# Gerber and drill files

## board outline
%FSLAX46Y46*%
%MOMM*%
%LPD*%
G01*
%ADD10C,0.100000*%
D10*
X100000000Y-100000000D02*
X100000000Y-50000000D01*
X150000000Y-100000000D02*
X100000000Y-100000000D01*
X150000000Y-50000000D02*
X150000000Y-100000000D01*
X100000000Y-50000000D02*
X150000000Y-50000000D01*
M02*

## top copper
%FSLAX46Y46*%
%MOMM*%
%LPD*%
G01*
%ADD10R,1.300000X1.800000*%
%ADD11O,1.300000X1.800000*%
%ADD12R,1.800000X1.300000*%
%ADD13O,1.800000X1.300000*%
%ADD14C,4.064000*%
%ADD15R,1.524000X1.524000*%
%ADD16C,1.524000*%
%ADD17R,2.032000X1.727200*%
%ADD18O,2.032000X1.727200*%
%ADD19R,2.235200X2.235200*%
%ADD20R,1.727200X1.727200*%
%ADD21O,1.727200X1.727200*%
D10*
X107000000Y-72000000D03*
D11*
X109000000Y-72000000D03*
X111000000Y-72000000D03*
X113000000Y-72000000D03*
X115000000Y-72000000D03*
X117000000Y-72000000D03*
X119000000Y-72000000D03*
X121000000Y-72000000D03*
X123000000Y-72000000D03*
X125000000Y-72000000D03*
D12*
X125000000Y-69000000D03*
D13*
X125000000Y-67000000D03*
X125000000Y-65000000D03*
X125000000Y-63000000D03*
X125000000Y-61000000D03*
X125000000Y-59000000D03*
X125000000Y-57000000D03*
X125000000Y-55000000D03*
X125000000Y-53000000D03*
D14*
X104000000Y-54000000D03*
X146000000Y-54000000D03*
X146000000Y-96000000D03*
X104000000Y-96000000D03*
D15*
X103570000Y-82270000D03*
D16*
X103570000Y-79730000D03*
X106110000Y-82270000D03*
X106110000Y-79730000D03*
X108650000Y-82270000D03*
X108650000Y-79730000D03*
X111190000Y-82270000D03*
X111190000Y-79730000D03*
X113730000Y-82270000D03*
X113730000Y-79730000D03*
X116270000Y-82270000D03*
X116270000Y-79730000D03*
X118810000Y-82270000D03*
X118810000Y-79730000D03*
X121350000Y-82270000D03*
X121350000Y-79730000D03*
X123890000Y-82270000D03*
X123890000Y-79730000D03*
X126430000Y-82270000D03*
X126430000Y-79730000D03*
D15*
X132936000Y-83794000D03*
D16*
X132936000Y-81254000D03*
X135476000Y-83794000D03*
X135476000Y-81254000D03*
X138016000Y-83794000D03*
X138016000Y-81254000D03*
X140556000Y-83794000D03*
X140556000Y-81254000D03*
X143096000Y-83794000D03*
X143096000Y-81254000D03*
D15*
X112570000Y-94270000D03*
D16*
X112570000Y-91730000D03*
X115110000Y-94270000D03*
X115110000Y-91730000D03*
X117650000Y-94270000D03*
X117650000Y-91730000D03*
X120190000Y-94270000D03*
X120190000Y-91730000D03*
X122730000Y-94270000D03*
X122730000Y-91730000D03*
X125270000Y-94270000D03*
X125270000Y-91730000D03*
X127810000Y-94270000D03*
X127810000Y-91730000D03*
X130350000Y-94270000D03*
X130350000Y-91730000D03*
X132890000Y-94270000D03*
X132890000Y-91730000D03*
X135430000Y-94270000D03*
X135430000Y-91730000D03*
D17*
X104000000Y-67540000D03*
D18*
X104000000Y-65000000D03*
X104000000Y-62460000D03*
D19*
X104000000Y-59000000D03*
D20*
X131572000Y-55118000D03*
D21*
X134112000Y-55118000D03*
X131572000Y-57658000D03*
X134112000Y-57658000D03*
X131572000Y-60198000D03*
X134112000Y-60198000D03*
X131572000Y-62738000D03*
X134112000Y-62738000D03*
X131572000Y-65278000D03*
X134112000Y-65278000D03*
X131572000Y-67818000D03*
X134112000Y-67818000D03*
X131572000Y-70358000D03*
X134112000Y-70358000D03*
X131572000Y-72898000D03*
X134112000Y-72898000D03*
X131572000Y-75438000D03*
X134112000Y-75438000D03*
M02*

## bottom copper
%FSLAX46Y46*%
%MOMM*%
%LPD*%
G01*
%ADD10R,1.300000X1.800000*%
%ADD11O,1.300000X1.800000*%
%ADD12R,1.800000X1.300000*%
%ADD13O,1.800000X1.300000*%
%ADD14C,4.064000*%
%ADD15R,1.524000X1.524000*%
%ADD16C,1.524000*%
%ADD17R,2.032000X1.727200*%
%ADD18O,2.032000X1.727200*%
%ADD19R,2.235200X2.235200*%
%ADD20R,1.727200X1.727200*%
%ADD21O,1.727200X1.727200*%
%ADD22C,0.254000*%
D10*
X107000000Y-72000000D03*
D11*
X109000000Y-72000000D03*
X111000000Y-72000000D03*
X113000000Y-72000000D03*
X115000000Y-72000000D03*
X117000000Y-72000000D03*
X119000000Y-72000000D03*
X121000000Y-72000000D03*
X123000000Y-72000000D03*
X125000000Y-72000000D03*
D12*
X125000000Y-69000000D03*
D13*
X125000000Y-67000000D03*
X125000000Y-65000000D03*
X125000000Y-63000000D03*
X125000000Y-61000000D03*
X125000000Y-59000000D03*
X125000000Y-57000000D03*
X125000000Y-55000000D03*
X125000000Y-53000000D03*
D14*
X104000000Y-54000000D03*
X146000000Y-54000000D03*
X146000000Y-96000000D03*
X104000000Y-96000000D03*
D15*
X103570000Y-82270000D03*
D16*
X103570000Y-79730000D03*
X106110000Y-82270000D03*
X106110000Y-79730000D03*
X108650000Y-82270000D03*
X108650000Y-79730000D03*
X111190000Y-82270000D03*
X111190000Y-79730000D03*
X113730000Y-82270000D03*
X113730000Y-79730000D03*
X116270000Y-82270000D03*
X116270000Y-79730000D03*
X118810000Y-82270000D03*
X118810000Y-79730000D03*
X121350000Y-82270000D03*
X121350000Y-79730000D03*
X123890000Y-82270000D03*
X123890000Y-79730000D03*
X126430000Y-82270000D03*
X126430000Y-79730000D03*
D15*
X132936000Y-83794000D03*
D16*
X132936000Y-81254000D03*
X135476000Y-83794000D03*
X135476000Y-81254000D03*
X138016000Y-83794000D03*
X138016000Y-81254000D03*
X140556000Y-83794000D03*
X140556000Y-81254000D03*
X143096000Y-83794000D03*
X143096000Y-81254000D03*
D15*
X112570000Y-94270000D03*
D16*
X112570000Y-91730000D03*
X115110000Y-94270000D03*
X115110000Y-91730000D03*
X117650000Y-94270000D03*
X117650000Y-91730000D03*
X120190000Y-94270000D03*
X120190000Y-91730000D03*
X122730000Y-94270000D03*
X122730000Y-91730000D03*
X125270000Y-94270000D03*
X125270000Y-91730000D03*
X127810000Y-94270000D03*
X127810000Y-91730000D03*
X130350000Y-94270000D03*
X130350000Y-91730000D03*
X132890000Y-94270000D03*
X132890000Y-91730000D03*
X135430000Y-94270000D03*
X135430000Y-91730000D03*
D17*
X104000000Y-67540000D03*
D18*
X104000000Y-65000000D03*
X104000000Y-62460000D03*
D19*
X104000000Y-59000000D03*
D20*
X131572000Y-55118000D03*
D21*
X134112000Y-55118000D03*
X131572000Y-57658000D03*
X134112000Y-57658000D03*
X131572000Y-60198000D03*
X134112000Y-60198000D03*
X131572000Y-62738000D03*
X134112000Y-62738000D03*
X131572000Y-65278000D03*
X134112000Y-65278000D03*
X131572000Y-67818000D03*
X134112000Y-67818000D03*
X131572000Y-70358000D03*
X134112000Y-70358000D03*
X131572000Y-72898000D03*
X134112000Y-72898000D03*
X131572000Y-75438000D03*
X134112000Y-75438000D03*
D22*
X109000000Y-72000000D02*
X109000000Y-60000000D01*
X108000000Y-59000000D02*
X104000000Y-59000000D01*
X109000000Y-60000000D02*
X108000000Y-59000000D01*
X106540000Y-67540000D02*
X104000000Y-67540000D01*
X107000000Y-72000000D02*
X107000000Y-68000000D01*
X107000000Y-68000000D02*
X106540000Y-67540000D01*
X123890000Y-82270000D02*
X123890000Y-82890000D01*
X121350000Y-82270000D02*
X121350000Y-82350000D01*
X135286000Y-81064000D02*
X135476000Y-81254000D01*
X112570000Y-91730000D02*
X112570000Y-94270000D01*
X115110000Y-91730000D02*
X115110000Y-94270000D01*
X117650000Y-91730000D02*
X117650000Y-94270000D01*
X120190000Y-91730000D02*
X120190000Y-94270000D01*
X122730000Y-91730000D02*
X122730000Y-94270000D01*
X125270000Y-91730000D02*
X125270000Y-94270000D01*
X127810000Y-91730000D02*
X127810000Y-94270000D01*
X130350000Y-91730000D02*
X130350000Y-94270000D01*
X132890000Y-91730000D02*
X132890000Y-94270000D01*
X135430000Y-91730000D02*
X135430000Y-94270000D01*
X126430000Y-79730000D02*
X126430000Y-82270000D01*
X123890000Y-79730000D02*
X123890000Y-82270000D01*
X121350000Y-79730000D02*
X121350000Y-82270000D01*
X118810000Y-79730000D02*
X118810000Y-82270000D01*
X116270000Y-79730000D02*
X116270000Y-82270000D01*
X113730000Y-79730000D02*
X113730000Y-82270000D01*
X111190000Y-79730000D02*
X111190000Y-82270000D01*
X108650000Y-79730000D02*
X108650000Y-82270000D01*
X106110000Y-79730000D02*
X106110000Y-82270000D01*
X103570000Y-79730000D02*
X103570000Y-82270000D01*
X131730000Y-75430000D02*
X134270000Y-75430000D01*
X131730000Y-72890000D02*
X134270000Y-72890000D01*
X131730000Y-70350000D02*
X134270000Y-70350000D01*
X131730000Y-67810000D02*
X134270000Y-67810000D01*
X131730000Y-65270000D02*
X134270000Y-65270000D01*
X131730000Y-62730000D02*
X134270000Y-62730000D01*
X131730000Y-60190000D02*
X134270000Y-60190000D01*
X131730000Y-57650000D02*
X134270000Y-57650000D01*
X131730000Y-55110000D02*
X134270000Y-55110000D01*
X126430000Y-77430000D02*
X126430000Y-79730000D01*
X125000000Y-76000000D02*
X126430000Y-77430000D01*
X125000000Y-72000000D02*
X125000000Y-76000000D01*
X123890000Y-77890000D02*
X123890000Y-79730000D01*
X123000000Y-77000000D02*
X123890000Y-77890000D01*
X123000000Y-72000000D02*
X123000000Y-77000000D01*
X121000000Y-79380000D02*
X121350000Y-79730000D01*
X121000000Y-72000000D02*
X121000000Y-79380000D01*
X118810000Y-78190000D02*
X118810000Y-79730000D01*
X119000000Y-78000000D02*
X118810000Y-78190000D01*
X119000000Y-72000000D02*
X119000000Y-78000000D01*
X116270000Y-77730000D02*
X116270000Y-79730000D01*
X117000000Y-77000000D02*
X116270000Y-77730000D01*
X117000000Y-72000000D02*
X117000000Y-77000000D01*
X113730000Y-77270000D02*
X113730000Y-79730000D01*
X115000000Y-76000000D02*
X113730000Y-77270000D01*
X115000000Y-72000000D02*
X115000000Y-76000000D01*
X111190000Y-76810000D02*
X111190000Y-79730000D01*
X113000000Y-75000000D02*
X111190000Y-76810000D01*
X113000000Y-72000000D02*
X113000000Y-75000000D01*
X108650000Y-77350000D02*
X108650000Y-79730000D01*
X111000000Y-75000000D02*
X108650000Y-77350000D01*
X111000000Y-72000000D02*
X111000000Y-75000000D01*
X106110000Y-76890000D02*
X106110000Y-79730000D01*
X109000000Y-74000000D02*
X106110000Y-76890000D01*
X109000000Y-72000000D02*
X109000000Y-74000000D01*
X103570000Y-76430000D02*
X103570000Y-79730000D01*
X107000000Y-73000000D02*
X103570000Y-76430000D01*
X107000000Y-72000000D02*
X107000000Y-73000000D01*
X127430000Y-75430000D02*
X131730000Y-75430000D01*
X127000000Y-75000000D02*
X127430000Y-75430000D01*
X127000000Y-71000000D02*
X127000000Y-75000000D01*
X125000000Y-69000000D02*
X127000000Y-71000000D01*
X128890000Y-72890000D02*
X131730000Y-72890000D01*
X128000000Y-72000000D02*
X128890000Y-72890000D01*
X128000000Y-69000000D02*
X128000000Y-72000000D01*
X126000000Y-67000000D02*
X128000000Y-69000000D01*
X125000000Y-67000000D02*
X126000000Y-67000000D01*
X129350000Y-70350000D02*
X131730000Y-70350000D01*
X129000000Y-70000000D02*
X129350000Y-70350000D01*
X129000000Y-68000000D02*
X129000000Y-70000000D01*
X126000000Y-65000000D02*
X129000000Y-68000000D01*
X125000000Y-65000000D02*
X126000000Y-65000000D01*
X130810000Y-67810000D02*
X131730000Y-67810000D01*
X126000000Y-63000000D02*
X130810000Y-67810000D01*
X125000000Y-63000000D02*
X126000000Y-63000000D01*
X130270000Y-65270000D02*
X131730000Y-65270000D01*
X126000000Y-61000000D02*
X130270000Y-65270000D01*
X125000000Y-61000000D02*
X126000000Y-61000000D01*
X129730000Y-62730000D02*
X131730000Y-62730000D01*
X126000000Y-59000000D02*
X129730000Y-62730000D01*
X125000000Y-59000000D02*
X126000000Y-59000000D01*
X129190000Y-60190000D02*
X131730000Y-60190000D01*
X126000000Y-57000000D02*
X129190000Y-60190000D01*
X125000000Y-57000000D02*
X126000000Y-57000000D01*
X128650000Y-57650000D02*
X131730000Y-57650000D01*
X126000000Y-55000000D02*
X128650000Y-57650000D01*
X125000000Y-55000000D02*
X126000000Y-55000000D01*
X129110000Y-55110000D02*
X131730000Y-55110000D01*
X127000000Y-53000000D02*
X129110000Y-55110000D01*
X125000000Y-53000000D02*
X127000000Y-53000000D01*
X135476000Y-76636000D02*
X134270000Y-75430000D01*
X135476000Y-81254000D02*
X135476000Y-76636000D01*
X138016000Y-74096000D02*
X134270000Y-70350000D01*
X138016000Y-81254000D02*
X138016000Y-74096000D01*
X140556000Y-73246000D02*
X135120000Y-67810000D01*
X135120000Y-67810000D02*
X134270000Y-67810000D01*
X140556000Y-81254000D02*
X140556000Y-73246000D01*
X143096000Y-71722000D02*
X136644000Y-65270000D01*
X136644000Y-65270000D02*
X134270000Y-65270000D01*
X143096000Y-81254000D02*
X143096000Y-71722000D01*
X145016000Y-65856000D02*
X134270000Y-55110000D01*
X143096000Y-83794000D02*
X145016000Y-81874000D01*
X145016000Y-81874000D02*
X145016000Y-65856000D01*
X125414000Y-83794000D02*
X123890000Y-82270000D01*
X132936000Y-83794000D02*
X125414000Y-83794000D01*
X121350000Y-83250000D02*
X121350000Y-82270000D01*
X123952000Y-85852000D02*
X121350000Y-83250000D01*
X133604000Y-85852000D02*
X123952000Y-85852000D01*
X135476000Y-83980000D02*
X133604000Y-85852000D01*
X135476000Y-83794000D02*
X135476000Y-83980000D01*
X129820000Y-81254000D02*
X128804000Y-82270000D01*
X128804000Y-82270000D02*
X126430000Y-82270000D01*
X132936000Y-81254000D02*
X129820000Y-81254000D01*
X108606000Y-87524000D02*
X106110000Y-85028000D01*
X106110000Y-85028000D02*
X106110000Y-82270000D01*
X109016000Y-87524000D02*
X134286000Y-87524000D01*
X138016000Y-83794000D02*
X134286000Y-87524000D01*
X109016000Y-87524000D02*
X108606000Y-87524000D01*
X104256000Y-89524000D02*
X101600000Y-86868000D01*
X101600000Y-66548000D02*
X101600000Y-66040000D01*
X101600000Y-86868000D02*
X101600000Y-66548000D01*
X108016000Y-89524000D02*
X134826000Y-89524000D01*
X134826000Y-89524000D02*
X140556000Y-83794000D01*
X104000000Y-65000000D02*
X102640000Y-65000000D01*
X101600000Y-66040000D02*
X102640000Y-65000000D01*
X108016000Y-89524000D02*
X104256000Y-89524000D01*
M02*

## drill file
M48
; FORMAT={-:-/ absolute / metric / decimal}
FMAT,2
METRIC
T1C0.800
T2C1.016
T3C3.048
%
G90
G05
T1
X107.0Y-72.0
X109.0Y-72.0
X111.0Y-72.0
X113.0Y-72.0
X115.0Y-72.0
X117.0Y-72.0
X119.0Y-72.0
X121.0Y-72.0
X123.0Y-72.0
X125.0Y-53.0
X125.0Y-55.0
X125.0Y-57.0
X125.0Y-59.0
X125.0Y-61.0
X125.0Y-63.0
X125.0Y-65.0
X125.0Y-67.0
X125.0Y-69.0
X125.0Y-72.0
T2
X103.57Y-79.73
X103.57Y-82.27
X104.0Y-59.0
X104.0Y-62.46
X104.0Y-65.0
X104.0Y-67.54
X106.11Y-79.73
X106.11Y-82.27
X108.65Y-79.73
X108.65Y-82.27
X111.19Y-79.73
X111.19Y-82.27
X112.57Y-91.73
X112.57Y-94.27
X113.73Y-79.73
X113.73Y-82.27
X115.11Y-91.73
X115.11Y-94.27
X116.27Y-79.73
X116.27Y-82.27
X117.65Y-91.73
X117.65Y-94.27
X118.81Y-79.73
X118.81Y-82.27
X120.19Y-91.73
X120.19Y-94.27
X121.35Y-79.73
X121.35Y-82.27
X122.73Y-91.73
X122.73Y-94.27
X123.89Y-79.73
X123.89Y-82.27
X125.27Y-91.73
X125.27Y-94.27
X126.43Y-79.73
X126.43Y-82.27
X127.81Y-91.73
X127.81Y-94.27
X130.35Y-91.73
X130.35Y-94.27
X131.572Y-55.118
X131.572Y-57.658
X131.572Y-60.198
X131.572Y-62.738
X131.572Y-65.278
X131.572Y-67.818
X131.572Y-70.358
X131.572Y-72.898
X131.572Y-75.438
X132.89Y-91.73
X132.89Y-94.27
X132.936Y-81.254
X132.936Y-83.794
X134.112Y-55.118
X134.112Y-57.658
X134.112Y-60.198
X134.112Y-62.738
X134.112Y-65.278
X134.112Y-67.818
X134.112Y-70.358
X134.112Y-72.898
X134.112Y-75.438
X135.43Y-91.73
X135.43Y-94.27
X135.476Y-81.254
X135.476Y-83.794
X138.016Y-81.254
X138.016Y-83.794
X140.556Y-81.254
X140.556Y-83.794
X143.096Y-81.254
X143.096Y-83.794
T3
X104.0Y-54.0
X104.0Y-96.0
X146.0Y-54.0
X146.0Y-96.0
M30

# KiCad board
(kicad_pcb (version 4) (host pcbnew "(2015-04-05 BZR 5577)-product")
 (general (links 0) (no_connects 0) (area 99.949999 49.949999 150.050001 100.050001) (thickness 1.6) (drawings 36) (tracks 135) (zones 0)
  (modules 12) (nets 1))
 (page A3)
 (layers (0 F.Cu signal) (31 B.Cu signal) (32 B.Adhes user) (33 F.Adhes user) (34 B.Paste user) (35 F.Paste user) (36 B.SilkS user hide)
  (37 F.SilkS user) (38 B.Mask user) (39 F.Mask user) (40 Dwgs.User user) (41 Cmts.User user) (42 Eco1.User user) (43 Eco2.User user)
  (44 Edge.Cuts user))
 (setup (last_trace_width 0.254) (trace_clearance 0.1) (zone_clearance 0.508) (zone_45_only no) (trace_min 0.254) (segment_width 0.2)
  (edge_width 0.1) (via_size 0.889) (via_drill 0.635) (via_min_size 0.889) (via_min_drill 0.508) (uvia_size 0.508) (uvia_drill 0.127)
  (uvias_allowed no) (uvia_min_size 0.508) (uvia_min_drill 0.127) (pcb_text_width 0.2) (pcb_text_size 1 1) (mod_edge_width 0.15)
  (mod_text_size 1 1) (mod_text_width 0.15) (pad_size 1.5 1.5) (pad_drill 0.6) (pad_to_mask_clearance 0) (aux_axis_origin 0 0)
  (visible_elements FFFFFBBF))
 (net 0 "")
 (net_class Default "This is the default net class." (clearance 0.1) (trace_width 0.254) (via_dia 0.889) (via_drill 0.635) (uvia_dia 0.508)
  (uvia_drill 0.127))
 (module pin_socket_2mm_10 (layer F.Cu) (at 116 72)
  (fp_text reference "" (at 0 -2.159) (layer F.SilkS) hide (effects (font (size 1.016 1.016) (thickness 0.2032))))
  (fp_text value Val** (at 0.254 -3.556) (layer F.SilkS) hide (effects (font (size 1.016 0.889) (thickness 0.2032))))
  (pad 1 thru_hole rect (at -9 0) (size 1.3 1.8) (drill 0.8) (layers *.Cu *.Mask F.SilkS))
  (pad 2 thru_hole oval (at -7 0) (size 1.3 1.8) (drill 0.8) (layers *.Cu *.Mask F.SilkS))
  (pad 3 thru_hole oval (at -5 0) (size 1.3 1.8) (drill 0.8) (layers *.Cu *.Mask F.SilkS))
  (pad 4 thru_hole oval (at -3 0) (size 1.3 1.8) (drill 0.8) (layers *.Cu *.Mask F.SilkS))
  (pad 5 thru_hole oval (at -1 0) (size 1.3 1.8) (drill 0.8) (layers *.Cu *.Mask F.SilkS))
  (pad 6 thru_hole oval (at 1 0) (size 1.3 1.8) (drill 0.8) (layers *.Cu *.Mask F.SilkS))
  (pad 7 thru_hole oval (at 3 0) (size 1.3 1.8) (drill 0.8) (layers *.Cu *.Mask F.SilkS))
  (pad 8 thru_hole oval (at 5 0) (size 1.3 1.8) (drill 0.8) (layers *.Cu *.Mask F.SilkS))
  (pad 9 thru_hole oval (at 7 0) (size 1.3 1.8) (drill 0.8) (layers *.Cu *.Mask F.SilkS))
  (pad 10 thru_hole oval (at 9 0) (size 1.3 1.8) (drill 0.8) (layers *.Cu *.Mask F.SilkS)))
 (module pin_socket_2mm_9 (layer F.Cu) (at 125 61 90)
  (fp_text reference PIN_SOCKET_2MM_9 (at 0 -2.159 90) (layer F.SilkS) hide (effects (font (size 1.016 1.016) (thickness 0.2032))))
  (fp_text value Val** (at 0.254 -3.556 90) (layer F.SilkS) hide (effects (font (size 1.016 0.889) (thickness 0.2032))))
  (pad 1 thru_hole rect (at -8 0 90) (size 1.3 1.8) (drill 0.8) (layers *.Cu *.Mask F.SilkS))
  (pad 2 thru_hole oval (at -6 0 90) (size 1.3 1.8) (drill 0.8) (layers *.Cu *.Mask F.SilkS))
  (pad 3 thru_hole oval (at -4 0 90) (size 1.3 1.8) (drill 0.8) (layers *.Cu *.Mask F.SilkS))
  (pad 4 thru_hole oval (at -2 0 90) (size 1.3 1.8) (drill 0.8) (layers *.Cu *.Mask F.SilkS))
  (pad 5 thru_hole oval (at 0 0 90) (size 1.3 1.8) (drill 0.8) (layers *.Cu *.Mask F.SilkS))
  (pad 6 thru_hole oval (at 2 0 90) (size 1.3 1.8) (drill 0.8) (layers *.Cu *.Mask F.SilkS))
  (pad 7 thru_hole oval (at 4 0 90) (size 1.3 1.8) (drill 0.8) (layers *.Cu *.Mask F.SilkS))
  (pad 8 thru_hole oval (at 6 0 90) (size 1.3 1.8) (drill 0.8) (layers *.Cu *.Mask F.SilkS))
  (pad 9 thru_hole oval (at 8 0 90) (size 1.3 1.8) (drill 0.8) (layers *.Cu *.Mask F.SilkS)))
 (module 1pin (layer F.Cu) (at 104 54)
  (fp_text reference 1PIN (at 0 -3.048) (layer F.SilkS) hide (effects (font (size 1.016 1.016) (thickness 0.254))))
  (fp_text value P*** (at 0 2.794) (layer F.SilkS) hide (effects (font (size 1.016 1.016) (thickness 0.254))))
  (pad 1 thru_hole circle (at 0 0) (size 4.064 4.064) (drill 3.048) (layers *.Cu *.Mask F.SilkS)))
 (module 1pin (layer F.Cu) (at 146 54)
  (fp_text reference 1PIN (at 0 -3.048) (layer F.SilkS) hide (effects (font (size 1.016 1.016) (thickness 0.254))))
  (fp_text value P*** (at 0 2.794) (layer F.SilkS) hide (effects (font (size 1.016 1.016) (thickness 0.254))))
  (pad 1 thru_hole circle (at 0 0) (size 4.064 4.064) (drill 3.048) (layers *.Cu *.Mask F.SilkS)))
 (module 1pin (layer F.Cu) (at 146 96)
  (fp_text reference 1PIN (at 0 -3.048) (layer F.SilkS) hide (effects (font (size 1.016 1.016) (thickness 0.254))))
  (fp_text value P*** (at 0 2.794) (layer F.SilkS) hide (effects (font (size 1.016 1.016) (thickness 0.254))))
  (pad 1 thru_hole circle (at 0 0) (size 4.064 4.064) (drill 3.048) (layers *.Cu *.Mask F.SilkS)))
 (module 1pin (layer F.Cu) (at 104 96)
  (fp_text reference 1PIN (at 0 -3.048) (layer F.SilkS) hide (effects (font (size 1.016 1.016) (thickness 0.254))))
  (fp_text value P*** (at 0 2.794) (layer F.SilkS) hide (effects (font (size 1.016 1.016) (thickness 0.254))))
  (pad 1 thru_hole circle (at 0 0) (size 4.064 4.064) (drill 3.048) (layers *.Cu *.Mask F.SilkS)))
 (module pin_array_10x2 (layer F.Cu) (at 115 81)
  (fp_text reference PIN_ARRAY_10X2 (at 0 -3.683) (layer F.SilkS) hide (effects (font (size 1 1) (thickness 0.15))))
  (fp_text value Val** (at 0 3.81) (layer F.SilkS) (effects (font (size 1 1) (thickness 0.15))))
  (pad 1 thru_hole rect (at -11.43 1.27) (size 1.524 1.524) (drill 1.016) (layers *.Cu *.Mask F.SilkS))
  (pad 2 thru_hole circle (at -11.43 -1.27) (size 1.524 1.524) (drill 1.016) (layers *.Cu *.Mask F.SilkS))
  (pad 3 thru_hole circle (at -8.89 1.27) (size 1.524 1.524) (drill 1.016) (layers *.Cu *.Mask F.SilkS))
  (pad 4 thru_hole circle (at -8.89 -1.27) (size 1.524 1.524) (drill 1.016) (layers *.Cu *.Mask F.SilkS))
  (pad 5 thru_hole circle (at -6.35 1.27) (size 1.524 1.524) (drill 1.016) (layers *.Cu *.Mask F.SilkS))
  (pad 6 thru_hole circle (at -6.35 -1.27) (size 1.524 1.524) (drill 1.016) (layers *.Cu *.Mask F.SilkS))
  (pad 7 thru_hole circle (at -3.81 1.27) (size 1.524 1.524) (drill 1.016) (layers *.Cu *.Mask F.SilkS))
  (pad 8 thru_hole circle (at -3.81 -1.27) (size 1.524 1.524) (drill 1.016) (layers *.Cu *.Mask F.SilkS))
  (pad 9 thru_hole circle (at -1.27 1.27) (size 1.524 1.524) (drill 1.016) (layers *.Cu *.Mask F.SilkS))
  (pad 10 thru_hole circle (at -1.27 -1.27) (size 1.524 1.524) (drill 1.016) (layers *.Cu *.Mask F.SilkS))
  (pad 11 thru_hole circle (at 1.27 1.27) (size 1.524 1.524) (drill 1.016) (layers *.Cu *.Mask F.SilkS))
  (pad 12 thru_hole circle (at 1.27 -1.27) (size 1.524 1.524) (drill 1.016) (layers *.Cu *.Mask F.SilkS))
  (pad 13 thru_hole circle (at 3.81 1.27) (size 1.524 1.524) (drill 1.016) (layers *.Cu *.Mask F.SilkS))
  (pad 14 thru_hole circle (at 3.81 -1.27) (size 1.524 1.524) (drill 1.016) (layers *.Cu *.Mask F.SilkS))
  (pad 15 thru_hole circle (at 6.35 1.27) (size 1.524 1.524) (drill 1.016) (layers *.Cu *.Mask F.SilkS))
  (pad 16 thru_hole circle (at 6.35 -1.27) (size 1.524 1.524) (drill 1.016) (layers *.Cu *.Mask F.SilkS))
  (pad 17 thru_hole circle (at 8.89 1.27) (size 1.524 1.524) (drill 1.016) (layers *.Cu *.Mask F.SilkS))
  (pad 18 thru_hole circle (at 8.89 -1.27) (size 1.524 1.524) (drill 1.016) (layers *.Cu *.Mask F.SilkS))
  (pad 19 thru_hole circle (at 11.43 1.27) (size 1.524 1.524) (drill 1.016) (layers *.Cu *.Mask F.SilkS))
  (pad 20 thru_hole circle (at 11.43 -1.27) (size 1.524 1.524) (drill 1.016) (layers *.Cu *.Mask F.SilkS)))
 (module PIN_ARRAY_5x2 (layer F.Cu) (at 138.016 82.524)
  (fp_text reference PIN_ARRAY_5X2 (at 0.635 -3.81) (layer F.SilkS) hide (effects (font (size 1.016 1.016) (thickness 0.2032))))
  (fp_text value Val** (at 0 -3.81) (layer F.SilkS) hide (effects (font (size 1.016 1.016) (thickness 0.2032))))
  (pad 1 thru_hole rect (at -5.08 1.27) (size 1.524 1.524) (drill 1.016) (layers *.Cu *.Mask F.SilkS))
  (pad 2 thru_hole circle (at -5.08 -1.27) (size 1.524 1.524) (drill 1.016) (layers *.Cu *.Mask F.SilkS))
  (pad 3 thru_hole circle (at -2.54 1.27) (size 1.524 1.524) (drill 1.016) (layers *.Cu *.Mask F.SilkS))
  (pad 4 thru_hole circle (at -2.54 -1.27) (size 1.524 1.524) (drill 1.016) (layers *.Cu *.Mask F.SilkS))
  (pad 5 thru_hole circle (at 0 1.27) (size 1.524 1.524) (drill 1.016) (layers *.Cu *.Mask F.SilkS))
  (pad 6 thru_hole circle (at 0 -1.27) (size 1.524 1.524) (drill 1.016) (layers *.Cu *.Mask F.SilkS))
  (pad 7 thru_hole circle (at 2.54 1.27) (size 1.524 1.524) (drill 1.016) (layers *.Cu *.Mask F.SilkS))
  (pad 8 thru_hole circle (at 2.54 -1.27) (size 1.524 1.524) (drill 1.016) (layers *.Cu *.Mask F.SilkS))
  (pad 9 thru_hole circle (at 5.08 1.27) (size 1.524 1.524) (drill 1.016) (layers *.Cu *.Mask F.SilkS))
  (pad 10 thru_hole circle (at 5.08 -1.27) (size 1.524 1.524) (drill 1.016) (layers *.Cu *.Mask F.SilkS)))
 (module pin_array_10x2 (layer F.Cu) (at 124 93)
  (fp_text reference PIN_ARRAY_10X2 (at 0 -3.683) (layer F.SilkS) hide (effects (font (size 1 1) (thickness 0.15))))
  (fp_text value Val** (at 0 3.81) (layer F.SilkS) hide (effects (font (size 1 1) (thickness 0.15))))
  (pad 1 thru_hole rect (at -11.43 1.27) (size 1.524 1.524) (drill 1.016) (layers *.Cu *.Mask F.SilkS))
  (pad 2 thru_hole circle (at -11.43 -1.27) (size 1.524 1.524) (drill 1.016) (layers *.Cu *.Mask F.SilkS))
  (pad 3 thru_hole circle (at -8.89 1.27) (size 1.524 1.524) (drill 1.016) (layers *.Cu *.Mask F.SilkS))
  (pad 4 thru_hole circle (at -8.89 -1.27) (size 1.524 1.524) (drill 1.016) (layers *.Cu *.Mask F.SilkS))
  (pad 5 thru_hole circle (at -6.35 1.27) (size 1.524 1.524) (drill 1.016) (layers *.Cu *.Mask F.SilkS))
  (pad 6 thru_hole circle (at -6.35 -1.27) (size 1.524 1.524) (drill 1.016) (layers *.Cu *.Mask F.SilkS))
  (pad 7 thru_hole circle (at -3.81 1.27) (size 1.524 1.524) (drill 1.016) (layers *.Cu *.Mask F.SilkS))
  (pad 8 thru_hole circle (at -3.81 -1.27) (size 1.524 1.524) (drill 1.016) (layers *.Cu *.Mask F.SilkS))
  (pad 9 thru_hole circle (at -1.27 1.27) (size 1.524 1.524) (drill 1.016) (layers *.Cu *.Mask F.SilkS))
  (pad 10 thru_hole circle (at -1.27 -1.27) (size 1.524 1.524) (drill 1.016) (layers *.Cu *.Mask F.SilkS))
  (pad 11 thru_hole circle (at 1.27 1.27) (size 1.524 1.524) (drill 1.016) (layers *.Cu *.Mask F.SilkS))
  (pad 12 thru_hole circle (at 1.27 -1.27) (size 1.524 1.524) (drill 1.016) (layers *.Cu *.Mask F.SilkS))
  (pad 13 thru_hole circle (at 3.81 1.27) (size 1.524 1.524) (drill 1.016) (layers *.Cu *.Mask F.SilkS))
  (pad 14 thru_hole circle (at 3.81 -1.27) (size 1.524 1.524) (drill 1.016) (layers *.Cu *.Mask F.SilkS))
  (pad 15 thru_hole circle (at 6.35 1.27) (size 1.524 1.524) (drill 1.016) (layers *.Cu *.Mask F.SilkS))
  (pad 16 thru_hole circle (at 6.35 -1.27) (size 1.524 1.524) (drill 1.016) (layers *.Cu *.Mask F.SilkS))
  (pad 17 thru_hole circle (at 8.89 1.27) (size 1.524 1.524) (drill 1.016) (layers *.Cu *.Mask F.SilkS))
  (pad 18 thru_hole circle (at 8.89 -1.27) (size 1.524 1.524) (drill 1.016) (layers *.Cu *.Mask F.SilkS))
  (pad 19 thru_hole circle (at 11.43 1.27) (size 1.524 1.524) (drill 1.016) (layers *.Cu *.Mask F.SilkS))
  (pad 20 thru_hole circle (at 11.43 -1.27) (size 1.524 1.524) (drill 1.016) (layers *.Cu *.Mask F.SilkS)))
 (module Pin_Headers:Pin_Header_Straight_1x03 (layer F.Cu) (at 104 65 90)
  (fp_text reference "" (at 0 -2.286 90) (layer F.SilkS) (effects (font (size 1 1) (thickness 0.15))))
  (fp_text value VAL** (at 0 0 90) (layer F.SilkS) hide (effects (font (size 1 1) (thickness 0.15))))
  (pad 1 thru_hole rect (at -2.54 0 90) (size 1.7272 2.032) (drill 1.016) (layers *.Cu *.Mask F.SilkS))
  (pad 2 thru_hole oval (at 0 0 90) (size 1.7272 2.032) (drill 1.016) (layers *.Cu *.Mask F.SilkS))
  (pad 3 thru_hole oval (at 2.54 0 90) (size 1.7272 2.032) (drill 1.016) (layers *.Cu *.Mask F.SilkS)))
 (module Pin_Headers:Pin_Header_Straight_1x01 (layer F.Cu) (at 104 59)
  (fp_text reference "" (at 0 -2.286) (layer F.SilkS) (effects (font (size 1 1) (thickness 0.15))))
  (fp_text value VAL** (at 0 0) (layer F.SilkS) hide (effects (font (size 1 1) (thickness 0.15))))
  (pad 1 thru_hole rect (at 0 0) (size 2.2352 2.2352) (drill 1.016) (layers *.Cu *.Mask F.SilkS)))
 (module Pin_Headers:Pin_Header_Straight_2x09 (layer F.Cu) (at 131.572 55.118)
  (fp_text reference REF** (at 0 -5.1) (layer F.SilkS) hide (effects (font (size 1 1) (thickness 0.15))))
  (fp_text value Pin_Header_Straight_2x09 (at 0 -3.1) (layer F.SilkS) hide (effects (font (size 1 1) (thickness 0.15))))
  (pad 1 thru_hole rect (at 0 0) (size 1.7272 1.7272) (drill 1.016) (layers *.Cu *.Mask F.SilkS))
  (pad 2 thru_hole oval (at 2.54 0) (size 1.7272 1.7272) (drill 1.016) (layers *.Cu *.Mask F.SilkS))
  (pad 3 thru_hole oval (at 0 2.54) (size 1.7272 1.7272) (drill 1.016) (layers *.Cu *.Mask F.SilkS))
  (pad 4 thru_hole oval (at 2.54 2.54) (size 1.7272 1.7272) (drill 1.016) (layers *.Cu *.Mask F.SilkS))
  (pad 5 thru_hole oval (at 0 5.08) (size 1.7272 1.7272) (drill 1.016) (layers *.Cu *.Mask F.SilkS))
  (pad 6 thru_hole oval (at 2.54 5.08) (size 1.7272 1.7272) (drill 1.016) (layers *.Cu *.Mask F.SilkS))
  (pad 7 thru_hole oval (at 0 7.62) (size 1.7272 1.7272) (drill 1.016) (layers *.Cu *.Mask F.SilkS))
  (pad 8 thru_hole oval (at 2.54 7.62) (size 1.7272 1.7272) (drill 1.016) (layers *.Cu *.Mask F.SilkS))
  (pad 9 thru_hole oval (at 0 10.16) (size 1.7272 1.7272) (drill 1.016) (layers *.Cu *.Mask F.SilkS))
  (pad 10 thru_hole oval (at 2.54 10.16) (size 1.7272 1.7272) (drill 1.016) (layers *.Cu *.Mask F.SilkS))
  (pad 11 thru_hole oval (at 0 12.7) (size 1.7272 1.7272) (drill 1.016) (layers *.Cu *.Mask F.SilkS))
  (pad 12 thru_hole oval (at 2.54 12.7) (size 1.7272 1.7272) (drill 1.016) (layers *.Cu *.Mask F.SilkS))
  (pad 13 thru_hole oval (at 0 15.24) (size 1.7272 1.7272) (drill 1.016) (layers *.Cu *.Mask F.SilkS))
  (pad 14 thru_hole oval (at 2.54 15.24) (size 1.7272 1.7272) (drill 1.016) (layers *.Cu *.Mask F.SilkS))
  (pad 15 thru_hole oval (at 0 17.78) (size 1.7272 1.7272) (drill 1.016) (layers *.Cu *.Mask F.SilkS))
  (pad 16 thru_hole oval (at 2.54 17.78) (size 1.7272 1.7272) (drill 1.016) (layers *.Cu *.Mask F.SilkS))
  (pad 17 thru_hole oval (at 0 20.32) (size 1.7272 1.7272) (drill 1.016) (layers *.Cu *.Mask F.SilkS))
  (pad 18 thru_hole oval (at 2.54 20.32) (size 1.7272 1.7272) (drill 1.016) (layers *.Cu *.Mask F.SilkS)))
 (gr_line (start 100 100) (end 100 50) (angle 90) (layer Edge.Cuts) (width 0.1))
 (gr_line (start 150 100) (end 100 100) (angle 90) (layer Edge.Cuts) (width 0.1))
 (gr_line (start 150 50) (end 150 100) (angle 90) (layer Edge.Cuts) (width 0.1))
 (gr_line (start 100 50) (end 150 50) (angle 90) (layer Edge.Cuts) (width 0.1))
 (segment (start 109 72) (end 109 60) (width 0.254) (layer B.Cu) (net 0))
 (segment (start 108 59) (end 104 59) (width 0.254) (layer B.Cu) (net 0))
 (segment (start 109 60) (end 108 59) (width 0.254) (layer B.Cu) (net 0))
 (segment (start 106.54 67.54) (end 104 67.54) (width 0.254) (layer B.Cu) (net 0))
 (segment (start 107 72) (end 107 68) (width 0.254) (layer B.Cu) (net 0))
 (segment (start 107 68) (end 106.54 67.54) (width 0.254) (layer B.Cu) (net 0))
 (segment (start 123.89 82.27) (end 123.89 82.89) (width 0.254) (layer B.Cu) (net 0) (status 30))
 (segment (start 121.35 82.27) (end 121.35 82.35) (width 0.254) (layer B.Cu) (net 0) (status 30))
 (segment (start 135.286 81.064) (end 135.476 81.254) (width 0.254) (layer B.Cu) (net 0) (status 30))
 (segment (start 112.57 91.73) (end 112.57 94.27) (width 0.254) (layer B.Cu) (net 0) (status 30))
 (segment (start 115.11 91.73) (end 115.11 94.27) (width 0.254) (layer B.Cu) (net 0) (status 30))
 (segment (start 117.65 91.73) (end 117.65 94.27) (width 0.254) (layer B.Cu) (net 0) (status 30))
 (segment (start 120.19 91.73) (end 120.19 94.27) (width 0.254) (layer B.Cu) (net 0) (status 30))
 (segment (start 122.73 91.73) (end 122.73 94.27) (width 0.254) (layer B.Cu) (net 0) (status 30))
 (segment (start 125.27 91.73) (end 125.27 94.27) (width 0.254) (layer B.Cu) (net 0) (status 30))
 (segment (start 127.81 91.73) (end 127.81 94.27) (width 0.254) (layer B.Cu) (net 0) (status 30))
 (segment (start 130.35 91.73) (end 130.35 94.27) (width 0.254) (layer B.Cu) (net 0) (status 30))
 (segment (start 132.89 91.73) (end 132.89 94.27) (width 0.254) (layer B.Cu) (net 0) (status 30))
 (segment (start 135.43 91.73) (end 135.43 94.27) (width 0.254) (layer B.Cu) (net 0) (status 30))
 (segment (start 126.43 79.73) (end 126.43 82.27) (width 0.254) (layer B.Cu) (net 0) (status 30))
 (segment (start 123.89 79.73) (end 123.89 82.27) (width 0.254) (layer B.Cu) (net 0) (status 30))
 (segment (start 121.35 79.73) (end 121.35 82.27) (width 0.254) (layer B.Cu) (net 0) (status 30))
 (segment (start 118.81 79.73) (end 118.81 82.27) (width 0.254) (layer B.Cu) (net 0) (status 30))
 (segment (start 116.27 79.73) (end 116.27 82.27) (width 0.254) (layer B.Cu) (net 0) (status 30))
 (segment (start 113.73 79.73) (end 113.73 82.27) (width 0.254) (layer B.Cu) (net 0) (status 30))
 (segment (start 111.19 79.73) (end 111.19 82.27) (width 0.254) (layer B.Cu) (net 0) (status 30))
 (segment (start 108.65 79.73) (end 108.65 82.27) (width 0.254) (layer B.Cu) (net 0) (status 30))
 (segment (start 106.11 79.73) (end 106.11 82.27) (width 0.254) (layer B.Cu) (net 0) (status 30))
 (segment (start 103.57 79.73) (end 103.57 82.27) (width 0.254) (layer B.Cu) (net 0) (status 30))
 (segment (start 131.73 75.43) (end 134.27 75.43) (width 0.254) (layer B.Cu) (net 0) (status 30))
 (segment (start 131.73 72.89) (end 134.27 72.89) (width 0.254) (layer B.Cu) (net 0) (status 30))
 (segment (start 131.73 70.35) (end 134.27 70.35) (width 0.254) (layer B.Cu) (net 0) (status 30))
 (segment (start 131.73 67.81) (end 134.27 67.81) (width 0.254) (layer B.Cu) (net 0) (status 30))
 (segment (start 131.73 65.27) (end 134.27 65.27) (width 0.254) (layer B.Cu) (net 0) (status 30))
 (segment (start 131.73 62.73) (end 134.27 62.73) (width 0.254) (layer B.Cu) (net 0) (status 30))
 (segment (start 131.73 60.19) (end 134.27 60.19) (width 0.254) (layer B.Cu) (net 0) (status 30))
 (segment (start 131.73 57.65) (end 134.27 57.65) (width 0.254) (layer B.Cu) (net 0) (status 30))
 (segment (start 131.73 55.11) (end 134.27 55.11) (width 0.254) (layer B.Cu) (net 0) (status 30))
 (segment (start 126.43 77.43) (end 126.43 79.73) (width 0.254) (layer B.Cu) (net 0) (status 20))
 (segment (start 125 76) (end 126.43 77.43) (width 0.254) (layer B.Cu) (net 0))
 (segment (start 125 72) (end 125 76) (width 0.254) (layer B.Cu) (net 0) (status 10))
 (segment (start 123.89 77.89) (end 123.89 79.73) (width 0.254) (layer B.Cu) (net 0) (status 20))
 (segment (start 123 77) (end 123.89 77.89) (width 0.254) (layer B.Cu) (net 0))
 (segment (start 123 72) (end 123 77) (width 0.254) (layer B.Cu) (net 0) (status 10))
 (segment (start 121 79.38) (end 121.35 79.73) (width 0.254) (layer B.Cu) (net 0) (status 30))
 (segment (start 121 72) (end 121 79.38) (width 0.254) (layer B.Cu) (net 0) (status 30))
 (segment (start 118.81 78.19) (end 118.81 79.73) (width 0.254) (layer B.Cu) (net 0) (status 20))
 (segment (start 119 78) (end 118.81 78.19) (width 0.254) (layer B.Cu) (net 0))
 (segment (start 119 72) (end 119 78) (width 0.254) (layer B.Cu) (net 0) (status 10))
 (segment (start 116.27 77.73) (end 116.27 79.73) (width 0.254) (layer B.Cu) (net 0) (status 20))
 (segment (start 117 77) (end 116.27 77.73) (width 0.254) (layer B.Cu) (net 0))
 (segment (start 117 72) (end 117 77) (width 0.254) (layer B.Cu) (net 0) (status 10))
 (segment (start 113.73 77.27) (end 113.73 79.73) (width 0.254) (layer B.Cu) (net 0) (status 20))
 (segment (start 115 76) (end 113.73 77.27) (width 0.254) (layer B.Cu) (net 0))
 (segment (start 115 72) (end 115 76) (width 0.254) (layer B.Cu) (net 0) (status 10))
 (segment (start 111.19 76.81) (end 111.19 79.73) (width 0.254) (layer B.Cu) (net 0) (status 20))
 (segment (start 113 75) (end 111.19 76.81) (width 0.254) (layer B.Cu) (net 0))
 (segment (start 113 72) (end 113 75) (width 0.254) (layer B.Cu) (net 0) (status 10))
 (segment (start 108.65 77.35) (end 108.65 79.73) (width 0.254) (layer B.Cu) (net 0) (status 20))
 (segment (start 111 75) (end 108.65 77.35) (width 0.254) (layer B.Cu) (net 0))
 (segment (start 111 72) (end 111 75) (width 0.254) (layer B.Cu) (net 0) (status 10))
 (segment (start 106.11 76.89) (end 106.11 79.73) (width 0.254) (layer B.Cu) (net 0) (status 20))
 (segment (start 109 74) (end 106.11 76.89) (width 0.254) (layer B.Cu) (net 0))
 (segment (start 109 72) (end 109 74) (width 0.254) (layer B.Cu) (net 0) (status 10))
 (segment (start 103.57 76.43) (end 103.57 79.73) (width 0.254) (layer B.Cu) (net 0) (status 20))
 (segment (start 107 73) (end 103.57 76.43) (width 0.254) (layer B.Cu) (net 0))
 (segment (start 107 72) (end 107 73) (width 0.254) (layer B.Cu) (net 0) (status 10))
 (segment (start 127.43 75.43) (end 131.73 75.43) (width 0.254) (layer B.Cu) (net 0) (status 20))
 (segment (start 127 75) (end 127.43 75.43) (width 0.254) (layer B.Cu) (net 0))
 (segment (start 127 71) (end 127 75) (width 0.254) (layer B.Cu) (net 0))
 (segment (start 125 69) (end 127 71) (width 0.254) (layer B.Cu) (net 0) (status 10))
 (segment (start 128.89 72.89) (end 131.73 72.89) (width 0.254) (layer B.Cu) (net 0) (status 20))
 (segment (start 128 72) (end 128.89 72.89) (width 0.254) (layer B.Cu) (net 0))
 (segment (start 128 69) (end 128 72) (width 0.254) (layer B.Cu) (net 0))
 (segment (start 126 67) (end 128 69) (width 0.254) (layer B.Cu) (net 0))
 (segment (start 125 67) (end 126 67) (width 0.254) (layer B.Cu) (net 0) (status 10))
 (segment (start 129.35 70.35) (end 131.73 70.35) (width 0.254) (layer B.Cu) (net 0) (status 20))
 (segment (start 129 70) (end 129.35 70.35) (width 0.254) (layer B.Cu) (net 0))
 (segment (start 129 68) (end 129 70) (width 0.254) (layer B.Cu) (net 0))
 (segment (start 126 65) (end 129 68) (width 0.254) (layer B.Cu) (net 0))
 (segment (start 125 65) (end 126 65) (width 0.254) (layer B.Cu) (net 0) (status 10))
 (segment (start 130.81 67.81) (end 131.73 67.81) (width 0.254) (layer B.Cu) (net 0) (status 20))
 (segment (start 126 63) (end 130.81 67.81) (width 0.254) (layer B.Cu) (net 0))
 (segment (start 125 63) (end 126 63) (width 0.254) (layer B.Cu) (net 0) (status 10))
 (segment (start 130.27 65.27) (end 131.73 65.27) (width 0.254) (layer B.Cu) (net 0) (status 20))
 (segment (start 126 61) (end 130.27 65.27) (width 0.254) (layer B.Cu) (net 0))
 (segment (start 125 61) (end 126 61) (width 0.254) (layer B.Cu) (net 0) (status 10))
 (segment (start 129.73 62.73) (end 131.73 62.73) (width 0.254) (layer B.Cu) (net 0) (status 20))
 (segment (start 126 59) (end 129.73 62.73) (width 0.254) (layer B.Cu) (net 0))
 (segment (start 125 59) (end 126 59) (width 0.254) (layer B.Cu) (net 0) (status 10))
 (segment (start 129.19 60.19) (end 131.73 60.19) (width 0.254) (layer B.Cu) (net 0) (status 20))
 (segment (start 126 57) (end 129.19 60.19) (width 0.254) (layer B.Cu) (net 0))
 (segment (start 125 57) (end 126 57) (width 0.254) (layer B.Cu) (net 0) (status 10))
 (segment (start 128.65 57.65) (end 131.73 57.65) (width 0.254) (layer B.Cu) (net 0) (status 20))
 (segment (start 126 55) (end 128.65 57.65) (width 0.254) (layer B.Cu) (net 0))
 (segment (start 125 55) (end 126 55) (width 0.254) (layer B.Cu) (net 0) (status 10))
 (segment (start 129.11 55.11) (end 131.73 55.11) (width 0.254) (layer B.Cu) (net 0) (status 20))
 (segment (start 127 53) (end 129.11 55.11) (width 0.254) (layer B.Cu) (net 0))
 (segment (start 125 53) (end 127 53) (width 0.254) (layer B.Cu) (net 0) (status 10))
 (segment (start 135.476 76.636) (end 134.27 75.43) (width 0.254) (layer B.Cu) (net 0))
 (segment (start 135.476 81.254) (end 135.476 76.636) (width 0.254) (layer B.Cu) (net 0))
 (segment (start 138.016 74.096) (end 134.27 70.35) (width 0.254) (layer B.Cu) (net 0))
 (segment (start 138.016 81.254) (end 138.016 74.096) (width 0.254) (layer B.Cu) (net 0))
 (segment (start 140.556 73.246) (end 135.12 67.81) (width 0.254) (layer B.Cu) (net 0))
 (segment (start 135.12 67.81) (end 134.27 67.81) (width 0.254) (layer B.Cu) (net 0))
 (segment (start 140.556 81.254) (end 140.556 73.246) (width 0.254) (layer B.Cu) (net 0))
 (segment (start 143.096 71.722) (end 136.644 65.27) (width 0.254) (layer B.Cu) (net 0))
 (segment (start 136.644 65.27) (end 134.27 65.27) (width 0.254) (layer B.Cu) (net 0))
 (segment (start 143.096 81.254) (end 143.096 71.722) (width 0.254) (layer B.Cu) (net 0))
 (segment (start 145.016 65.856) (end 134.27 55.11) (width 0.254) (layer B.Cu) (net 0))
 (segment (start 143.096 83.794) (end 145.016 81.874) (width 0.254) (layer B.Cu) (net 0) (status 20))
 (segment (start 145.016 81.874) (end 145.016 65.856) (width 0.254) (layer B.Cu) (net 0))
 (segment (start 125.414 83.794) (end 123.89 82.27) (width 0.254) (layer B.Cu) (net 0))
 (segment (start 132.936 83.794) (end 125.414 83.794) (width 0.254) (layer B.Cu) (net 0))
 (segment (start 121.35 83.25) (end 121.35 82.27) (width 0.254) (layer B.Cu) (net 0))
 (segment (start 123.952 85.852) (end 121.35 83.25) (width 0.254) (layer B.Cu) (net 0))
 (segment (start 133.604 85.852) (end 123.952 85.852) (width 0.254) (layer B.Cu) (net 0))
 (segment (start 135.476 83.98) (end 133.604 85.852) (width 0.254) (layer B.Cu) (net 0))
 (segment (start 135.476 83.794) (end 135.476 83.98) (width 0.254) (layer B.Cu) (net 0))
 (segment (start 129.82 81.254) (end 128.804 82.27) (width 0.254) (layer B.Cu) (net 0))
 (segment (start 128.804 82.27) (end 126.43 82.27) (width 0.254) (layer B.Cu) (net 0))
 (segment (start 132.936 81.254) (end 129.82 81.254) (width 0.254) (layer B.Cu) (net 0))
 (segment (start 108.606 87.524) (end 106.11 85.028) (width 0.254) (layer B.Cu) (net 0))
 (segment (start 106.11 85.028) (end 106.11 82.27) (width 0.254) (layer B.Cu) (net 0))
 (segment (start 109.016 87.524) (end 134.286 87.524) (width 0.254) (layer B.Cu) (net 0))
 (segment (start 138.016 83.794) (end 134.286 87.524) (width 0.254) (layer B.Cu) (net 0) (status 20))
 (segment (start 109.016 87.524) (end 108.606 87.524) (width 0.254) (layer B.Cu) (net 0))
 (segment (start 104.256 89.524) (end 101.6 86.868) (width 0.254) (layer B.Cu) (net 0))
 (segment (start 101.6 66.548) (end 101.6 66.04) (width 0.254) (layer B.Cu) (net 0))
 (segment (start 101.6 86.868) (end 101.6 66.548) (width 0.254) (layer B.Cu) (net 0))
 (segment (start 108.016 89.524) (end 134.826 89.524) (width 0.254) (layer B.Cu) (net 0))
 (segment (start 134.826 89.524) (end 140.556 83.794) (width 0.254) (layer B.Cu) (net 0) (status 20))
 (segment (start 104 65) (end 102.64 65) (width 0.254) (layer B.Cu) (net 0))
 (segment (start 101.6 66.04) (end 102.64 65) (width 0.254) (layer B.Cu) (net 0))
 (segment (start 108.016 89.524) (end 104.256 89.524) (width 0.254) (layer B.Cu) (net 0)))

